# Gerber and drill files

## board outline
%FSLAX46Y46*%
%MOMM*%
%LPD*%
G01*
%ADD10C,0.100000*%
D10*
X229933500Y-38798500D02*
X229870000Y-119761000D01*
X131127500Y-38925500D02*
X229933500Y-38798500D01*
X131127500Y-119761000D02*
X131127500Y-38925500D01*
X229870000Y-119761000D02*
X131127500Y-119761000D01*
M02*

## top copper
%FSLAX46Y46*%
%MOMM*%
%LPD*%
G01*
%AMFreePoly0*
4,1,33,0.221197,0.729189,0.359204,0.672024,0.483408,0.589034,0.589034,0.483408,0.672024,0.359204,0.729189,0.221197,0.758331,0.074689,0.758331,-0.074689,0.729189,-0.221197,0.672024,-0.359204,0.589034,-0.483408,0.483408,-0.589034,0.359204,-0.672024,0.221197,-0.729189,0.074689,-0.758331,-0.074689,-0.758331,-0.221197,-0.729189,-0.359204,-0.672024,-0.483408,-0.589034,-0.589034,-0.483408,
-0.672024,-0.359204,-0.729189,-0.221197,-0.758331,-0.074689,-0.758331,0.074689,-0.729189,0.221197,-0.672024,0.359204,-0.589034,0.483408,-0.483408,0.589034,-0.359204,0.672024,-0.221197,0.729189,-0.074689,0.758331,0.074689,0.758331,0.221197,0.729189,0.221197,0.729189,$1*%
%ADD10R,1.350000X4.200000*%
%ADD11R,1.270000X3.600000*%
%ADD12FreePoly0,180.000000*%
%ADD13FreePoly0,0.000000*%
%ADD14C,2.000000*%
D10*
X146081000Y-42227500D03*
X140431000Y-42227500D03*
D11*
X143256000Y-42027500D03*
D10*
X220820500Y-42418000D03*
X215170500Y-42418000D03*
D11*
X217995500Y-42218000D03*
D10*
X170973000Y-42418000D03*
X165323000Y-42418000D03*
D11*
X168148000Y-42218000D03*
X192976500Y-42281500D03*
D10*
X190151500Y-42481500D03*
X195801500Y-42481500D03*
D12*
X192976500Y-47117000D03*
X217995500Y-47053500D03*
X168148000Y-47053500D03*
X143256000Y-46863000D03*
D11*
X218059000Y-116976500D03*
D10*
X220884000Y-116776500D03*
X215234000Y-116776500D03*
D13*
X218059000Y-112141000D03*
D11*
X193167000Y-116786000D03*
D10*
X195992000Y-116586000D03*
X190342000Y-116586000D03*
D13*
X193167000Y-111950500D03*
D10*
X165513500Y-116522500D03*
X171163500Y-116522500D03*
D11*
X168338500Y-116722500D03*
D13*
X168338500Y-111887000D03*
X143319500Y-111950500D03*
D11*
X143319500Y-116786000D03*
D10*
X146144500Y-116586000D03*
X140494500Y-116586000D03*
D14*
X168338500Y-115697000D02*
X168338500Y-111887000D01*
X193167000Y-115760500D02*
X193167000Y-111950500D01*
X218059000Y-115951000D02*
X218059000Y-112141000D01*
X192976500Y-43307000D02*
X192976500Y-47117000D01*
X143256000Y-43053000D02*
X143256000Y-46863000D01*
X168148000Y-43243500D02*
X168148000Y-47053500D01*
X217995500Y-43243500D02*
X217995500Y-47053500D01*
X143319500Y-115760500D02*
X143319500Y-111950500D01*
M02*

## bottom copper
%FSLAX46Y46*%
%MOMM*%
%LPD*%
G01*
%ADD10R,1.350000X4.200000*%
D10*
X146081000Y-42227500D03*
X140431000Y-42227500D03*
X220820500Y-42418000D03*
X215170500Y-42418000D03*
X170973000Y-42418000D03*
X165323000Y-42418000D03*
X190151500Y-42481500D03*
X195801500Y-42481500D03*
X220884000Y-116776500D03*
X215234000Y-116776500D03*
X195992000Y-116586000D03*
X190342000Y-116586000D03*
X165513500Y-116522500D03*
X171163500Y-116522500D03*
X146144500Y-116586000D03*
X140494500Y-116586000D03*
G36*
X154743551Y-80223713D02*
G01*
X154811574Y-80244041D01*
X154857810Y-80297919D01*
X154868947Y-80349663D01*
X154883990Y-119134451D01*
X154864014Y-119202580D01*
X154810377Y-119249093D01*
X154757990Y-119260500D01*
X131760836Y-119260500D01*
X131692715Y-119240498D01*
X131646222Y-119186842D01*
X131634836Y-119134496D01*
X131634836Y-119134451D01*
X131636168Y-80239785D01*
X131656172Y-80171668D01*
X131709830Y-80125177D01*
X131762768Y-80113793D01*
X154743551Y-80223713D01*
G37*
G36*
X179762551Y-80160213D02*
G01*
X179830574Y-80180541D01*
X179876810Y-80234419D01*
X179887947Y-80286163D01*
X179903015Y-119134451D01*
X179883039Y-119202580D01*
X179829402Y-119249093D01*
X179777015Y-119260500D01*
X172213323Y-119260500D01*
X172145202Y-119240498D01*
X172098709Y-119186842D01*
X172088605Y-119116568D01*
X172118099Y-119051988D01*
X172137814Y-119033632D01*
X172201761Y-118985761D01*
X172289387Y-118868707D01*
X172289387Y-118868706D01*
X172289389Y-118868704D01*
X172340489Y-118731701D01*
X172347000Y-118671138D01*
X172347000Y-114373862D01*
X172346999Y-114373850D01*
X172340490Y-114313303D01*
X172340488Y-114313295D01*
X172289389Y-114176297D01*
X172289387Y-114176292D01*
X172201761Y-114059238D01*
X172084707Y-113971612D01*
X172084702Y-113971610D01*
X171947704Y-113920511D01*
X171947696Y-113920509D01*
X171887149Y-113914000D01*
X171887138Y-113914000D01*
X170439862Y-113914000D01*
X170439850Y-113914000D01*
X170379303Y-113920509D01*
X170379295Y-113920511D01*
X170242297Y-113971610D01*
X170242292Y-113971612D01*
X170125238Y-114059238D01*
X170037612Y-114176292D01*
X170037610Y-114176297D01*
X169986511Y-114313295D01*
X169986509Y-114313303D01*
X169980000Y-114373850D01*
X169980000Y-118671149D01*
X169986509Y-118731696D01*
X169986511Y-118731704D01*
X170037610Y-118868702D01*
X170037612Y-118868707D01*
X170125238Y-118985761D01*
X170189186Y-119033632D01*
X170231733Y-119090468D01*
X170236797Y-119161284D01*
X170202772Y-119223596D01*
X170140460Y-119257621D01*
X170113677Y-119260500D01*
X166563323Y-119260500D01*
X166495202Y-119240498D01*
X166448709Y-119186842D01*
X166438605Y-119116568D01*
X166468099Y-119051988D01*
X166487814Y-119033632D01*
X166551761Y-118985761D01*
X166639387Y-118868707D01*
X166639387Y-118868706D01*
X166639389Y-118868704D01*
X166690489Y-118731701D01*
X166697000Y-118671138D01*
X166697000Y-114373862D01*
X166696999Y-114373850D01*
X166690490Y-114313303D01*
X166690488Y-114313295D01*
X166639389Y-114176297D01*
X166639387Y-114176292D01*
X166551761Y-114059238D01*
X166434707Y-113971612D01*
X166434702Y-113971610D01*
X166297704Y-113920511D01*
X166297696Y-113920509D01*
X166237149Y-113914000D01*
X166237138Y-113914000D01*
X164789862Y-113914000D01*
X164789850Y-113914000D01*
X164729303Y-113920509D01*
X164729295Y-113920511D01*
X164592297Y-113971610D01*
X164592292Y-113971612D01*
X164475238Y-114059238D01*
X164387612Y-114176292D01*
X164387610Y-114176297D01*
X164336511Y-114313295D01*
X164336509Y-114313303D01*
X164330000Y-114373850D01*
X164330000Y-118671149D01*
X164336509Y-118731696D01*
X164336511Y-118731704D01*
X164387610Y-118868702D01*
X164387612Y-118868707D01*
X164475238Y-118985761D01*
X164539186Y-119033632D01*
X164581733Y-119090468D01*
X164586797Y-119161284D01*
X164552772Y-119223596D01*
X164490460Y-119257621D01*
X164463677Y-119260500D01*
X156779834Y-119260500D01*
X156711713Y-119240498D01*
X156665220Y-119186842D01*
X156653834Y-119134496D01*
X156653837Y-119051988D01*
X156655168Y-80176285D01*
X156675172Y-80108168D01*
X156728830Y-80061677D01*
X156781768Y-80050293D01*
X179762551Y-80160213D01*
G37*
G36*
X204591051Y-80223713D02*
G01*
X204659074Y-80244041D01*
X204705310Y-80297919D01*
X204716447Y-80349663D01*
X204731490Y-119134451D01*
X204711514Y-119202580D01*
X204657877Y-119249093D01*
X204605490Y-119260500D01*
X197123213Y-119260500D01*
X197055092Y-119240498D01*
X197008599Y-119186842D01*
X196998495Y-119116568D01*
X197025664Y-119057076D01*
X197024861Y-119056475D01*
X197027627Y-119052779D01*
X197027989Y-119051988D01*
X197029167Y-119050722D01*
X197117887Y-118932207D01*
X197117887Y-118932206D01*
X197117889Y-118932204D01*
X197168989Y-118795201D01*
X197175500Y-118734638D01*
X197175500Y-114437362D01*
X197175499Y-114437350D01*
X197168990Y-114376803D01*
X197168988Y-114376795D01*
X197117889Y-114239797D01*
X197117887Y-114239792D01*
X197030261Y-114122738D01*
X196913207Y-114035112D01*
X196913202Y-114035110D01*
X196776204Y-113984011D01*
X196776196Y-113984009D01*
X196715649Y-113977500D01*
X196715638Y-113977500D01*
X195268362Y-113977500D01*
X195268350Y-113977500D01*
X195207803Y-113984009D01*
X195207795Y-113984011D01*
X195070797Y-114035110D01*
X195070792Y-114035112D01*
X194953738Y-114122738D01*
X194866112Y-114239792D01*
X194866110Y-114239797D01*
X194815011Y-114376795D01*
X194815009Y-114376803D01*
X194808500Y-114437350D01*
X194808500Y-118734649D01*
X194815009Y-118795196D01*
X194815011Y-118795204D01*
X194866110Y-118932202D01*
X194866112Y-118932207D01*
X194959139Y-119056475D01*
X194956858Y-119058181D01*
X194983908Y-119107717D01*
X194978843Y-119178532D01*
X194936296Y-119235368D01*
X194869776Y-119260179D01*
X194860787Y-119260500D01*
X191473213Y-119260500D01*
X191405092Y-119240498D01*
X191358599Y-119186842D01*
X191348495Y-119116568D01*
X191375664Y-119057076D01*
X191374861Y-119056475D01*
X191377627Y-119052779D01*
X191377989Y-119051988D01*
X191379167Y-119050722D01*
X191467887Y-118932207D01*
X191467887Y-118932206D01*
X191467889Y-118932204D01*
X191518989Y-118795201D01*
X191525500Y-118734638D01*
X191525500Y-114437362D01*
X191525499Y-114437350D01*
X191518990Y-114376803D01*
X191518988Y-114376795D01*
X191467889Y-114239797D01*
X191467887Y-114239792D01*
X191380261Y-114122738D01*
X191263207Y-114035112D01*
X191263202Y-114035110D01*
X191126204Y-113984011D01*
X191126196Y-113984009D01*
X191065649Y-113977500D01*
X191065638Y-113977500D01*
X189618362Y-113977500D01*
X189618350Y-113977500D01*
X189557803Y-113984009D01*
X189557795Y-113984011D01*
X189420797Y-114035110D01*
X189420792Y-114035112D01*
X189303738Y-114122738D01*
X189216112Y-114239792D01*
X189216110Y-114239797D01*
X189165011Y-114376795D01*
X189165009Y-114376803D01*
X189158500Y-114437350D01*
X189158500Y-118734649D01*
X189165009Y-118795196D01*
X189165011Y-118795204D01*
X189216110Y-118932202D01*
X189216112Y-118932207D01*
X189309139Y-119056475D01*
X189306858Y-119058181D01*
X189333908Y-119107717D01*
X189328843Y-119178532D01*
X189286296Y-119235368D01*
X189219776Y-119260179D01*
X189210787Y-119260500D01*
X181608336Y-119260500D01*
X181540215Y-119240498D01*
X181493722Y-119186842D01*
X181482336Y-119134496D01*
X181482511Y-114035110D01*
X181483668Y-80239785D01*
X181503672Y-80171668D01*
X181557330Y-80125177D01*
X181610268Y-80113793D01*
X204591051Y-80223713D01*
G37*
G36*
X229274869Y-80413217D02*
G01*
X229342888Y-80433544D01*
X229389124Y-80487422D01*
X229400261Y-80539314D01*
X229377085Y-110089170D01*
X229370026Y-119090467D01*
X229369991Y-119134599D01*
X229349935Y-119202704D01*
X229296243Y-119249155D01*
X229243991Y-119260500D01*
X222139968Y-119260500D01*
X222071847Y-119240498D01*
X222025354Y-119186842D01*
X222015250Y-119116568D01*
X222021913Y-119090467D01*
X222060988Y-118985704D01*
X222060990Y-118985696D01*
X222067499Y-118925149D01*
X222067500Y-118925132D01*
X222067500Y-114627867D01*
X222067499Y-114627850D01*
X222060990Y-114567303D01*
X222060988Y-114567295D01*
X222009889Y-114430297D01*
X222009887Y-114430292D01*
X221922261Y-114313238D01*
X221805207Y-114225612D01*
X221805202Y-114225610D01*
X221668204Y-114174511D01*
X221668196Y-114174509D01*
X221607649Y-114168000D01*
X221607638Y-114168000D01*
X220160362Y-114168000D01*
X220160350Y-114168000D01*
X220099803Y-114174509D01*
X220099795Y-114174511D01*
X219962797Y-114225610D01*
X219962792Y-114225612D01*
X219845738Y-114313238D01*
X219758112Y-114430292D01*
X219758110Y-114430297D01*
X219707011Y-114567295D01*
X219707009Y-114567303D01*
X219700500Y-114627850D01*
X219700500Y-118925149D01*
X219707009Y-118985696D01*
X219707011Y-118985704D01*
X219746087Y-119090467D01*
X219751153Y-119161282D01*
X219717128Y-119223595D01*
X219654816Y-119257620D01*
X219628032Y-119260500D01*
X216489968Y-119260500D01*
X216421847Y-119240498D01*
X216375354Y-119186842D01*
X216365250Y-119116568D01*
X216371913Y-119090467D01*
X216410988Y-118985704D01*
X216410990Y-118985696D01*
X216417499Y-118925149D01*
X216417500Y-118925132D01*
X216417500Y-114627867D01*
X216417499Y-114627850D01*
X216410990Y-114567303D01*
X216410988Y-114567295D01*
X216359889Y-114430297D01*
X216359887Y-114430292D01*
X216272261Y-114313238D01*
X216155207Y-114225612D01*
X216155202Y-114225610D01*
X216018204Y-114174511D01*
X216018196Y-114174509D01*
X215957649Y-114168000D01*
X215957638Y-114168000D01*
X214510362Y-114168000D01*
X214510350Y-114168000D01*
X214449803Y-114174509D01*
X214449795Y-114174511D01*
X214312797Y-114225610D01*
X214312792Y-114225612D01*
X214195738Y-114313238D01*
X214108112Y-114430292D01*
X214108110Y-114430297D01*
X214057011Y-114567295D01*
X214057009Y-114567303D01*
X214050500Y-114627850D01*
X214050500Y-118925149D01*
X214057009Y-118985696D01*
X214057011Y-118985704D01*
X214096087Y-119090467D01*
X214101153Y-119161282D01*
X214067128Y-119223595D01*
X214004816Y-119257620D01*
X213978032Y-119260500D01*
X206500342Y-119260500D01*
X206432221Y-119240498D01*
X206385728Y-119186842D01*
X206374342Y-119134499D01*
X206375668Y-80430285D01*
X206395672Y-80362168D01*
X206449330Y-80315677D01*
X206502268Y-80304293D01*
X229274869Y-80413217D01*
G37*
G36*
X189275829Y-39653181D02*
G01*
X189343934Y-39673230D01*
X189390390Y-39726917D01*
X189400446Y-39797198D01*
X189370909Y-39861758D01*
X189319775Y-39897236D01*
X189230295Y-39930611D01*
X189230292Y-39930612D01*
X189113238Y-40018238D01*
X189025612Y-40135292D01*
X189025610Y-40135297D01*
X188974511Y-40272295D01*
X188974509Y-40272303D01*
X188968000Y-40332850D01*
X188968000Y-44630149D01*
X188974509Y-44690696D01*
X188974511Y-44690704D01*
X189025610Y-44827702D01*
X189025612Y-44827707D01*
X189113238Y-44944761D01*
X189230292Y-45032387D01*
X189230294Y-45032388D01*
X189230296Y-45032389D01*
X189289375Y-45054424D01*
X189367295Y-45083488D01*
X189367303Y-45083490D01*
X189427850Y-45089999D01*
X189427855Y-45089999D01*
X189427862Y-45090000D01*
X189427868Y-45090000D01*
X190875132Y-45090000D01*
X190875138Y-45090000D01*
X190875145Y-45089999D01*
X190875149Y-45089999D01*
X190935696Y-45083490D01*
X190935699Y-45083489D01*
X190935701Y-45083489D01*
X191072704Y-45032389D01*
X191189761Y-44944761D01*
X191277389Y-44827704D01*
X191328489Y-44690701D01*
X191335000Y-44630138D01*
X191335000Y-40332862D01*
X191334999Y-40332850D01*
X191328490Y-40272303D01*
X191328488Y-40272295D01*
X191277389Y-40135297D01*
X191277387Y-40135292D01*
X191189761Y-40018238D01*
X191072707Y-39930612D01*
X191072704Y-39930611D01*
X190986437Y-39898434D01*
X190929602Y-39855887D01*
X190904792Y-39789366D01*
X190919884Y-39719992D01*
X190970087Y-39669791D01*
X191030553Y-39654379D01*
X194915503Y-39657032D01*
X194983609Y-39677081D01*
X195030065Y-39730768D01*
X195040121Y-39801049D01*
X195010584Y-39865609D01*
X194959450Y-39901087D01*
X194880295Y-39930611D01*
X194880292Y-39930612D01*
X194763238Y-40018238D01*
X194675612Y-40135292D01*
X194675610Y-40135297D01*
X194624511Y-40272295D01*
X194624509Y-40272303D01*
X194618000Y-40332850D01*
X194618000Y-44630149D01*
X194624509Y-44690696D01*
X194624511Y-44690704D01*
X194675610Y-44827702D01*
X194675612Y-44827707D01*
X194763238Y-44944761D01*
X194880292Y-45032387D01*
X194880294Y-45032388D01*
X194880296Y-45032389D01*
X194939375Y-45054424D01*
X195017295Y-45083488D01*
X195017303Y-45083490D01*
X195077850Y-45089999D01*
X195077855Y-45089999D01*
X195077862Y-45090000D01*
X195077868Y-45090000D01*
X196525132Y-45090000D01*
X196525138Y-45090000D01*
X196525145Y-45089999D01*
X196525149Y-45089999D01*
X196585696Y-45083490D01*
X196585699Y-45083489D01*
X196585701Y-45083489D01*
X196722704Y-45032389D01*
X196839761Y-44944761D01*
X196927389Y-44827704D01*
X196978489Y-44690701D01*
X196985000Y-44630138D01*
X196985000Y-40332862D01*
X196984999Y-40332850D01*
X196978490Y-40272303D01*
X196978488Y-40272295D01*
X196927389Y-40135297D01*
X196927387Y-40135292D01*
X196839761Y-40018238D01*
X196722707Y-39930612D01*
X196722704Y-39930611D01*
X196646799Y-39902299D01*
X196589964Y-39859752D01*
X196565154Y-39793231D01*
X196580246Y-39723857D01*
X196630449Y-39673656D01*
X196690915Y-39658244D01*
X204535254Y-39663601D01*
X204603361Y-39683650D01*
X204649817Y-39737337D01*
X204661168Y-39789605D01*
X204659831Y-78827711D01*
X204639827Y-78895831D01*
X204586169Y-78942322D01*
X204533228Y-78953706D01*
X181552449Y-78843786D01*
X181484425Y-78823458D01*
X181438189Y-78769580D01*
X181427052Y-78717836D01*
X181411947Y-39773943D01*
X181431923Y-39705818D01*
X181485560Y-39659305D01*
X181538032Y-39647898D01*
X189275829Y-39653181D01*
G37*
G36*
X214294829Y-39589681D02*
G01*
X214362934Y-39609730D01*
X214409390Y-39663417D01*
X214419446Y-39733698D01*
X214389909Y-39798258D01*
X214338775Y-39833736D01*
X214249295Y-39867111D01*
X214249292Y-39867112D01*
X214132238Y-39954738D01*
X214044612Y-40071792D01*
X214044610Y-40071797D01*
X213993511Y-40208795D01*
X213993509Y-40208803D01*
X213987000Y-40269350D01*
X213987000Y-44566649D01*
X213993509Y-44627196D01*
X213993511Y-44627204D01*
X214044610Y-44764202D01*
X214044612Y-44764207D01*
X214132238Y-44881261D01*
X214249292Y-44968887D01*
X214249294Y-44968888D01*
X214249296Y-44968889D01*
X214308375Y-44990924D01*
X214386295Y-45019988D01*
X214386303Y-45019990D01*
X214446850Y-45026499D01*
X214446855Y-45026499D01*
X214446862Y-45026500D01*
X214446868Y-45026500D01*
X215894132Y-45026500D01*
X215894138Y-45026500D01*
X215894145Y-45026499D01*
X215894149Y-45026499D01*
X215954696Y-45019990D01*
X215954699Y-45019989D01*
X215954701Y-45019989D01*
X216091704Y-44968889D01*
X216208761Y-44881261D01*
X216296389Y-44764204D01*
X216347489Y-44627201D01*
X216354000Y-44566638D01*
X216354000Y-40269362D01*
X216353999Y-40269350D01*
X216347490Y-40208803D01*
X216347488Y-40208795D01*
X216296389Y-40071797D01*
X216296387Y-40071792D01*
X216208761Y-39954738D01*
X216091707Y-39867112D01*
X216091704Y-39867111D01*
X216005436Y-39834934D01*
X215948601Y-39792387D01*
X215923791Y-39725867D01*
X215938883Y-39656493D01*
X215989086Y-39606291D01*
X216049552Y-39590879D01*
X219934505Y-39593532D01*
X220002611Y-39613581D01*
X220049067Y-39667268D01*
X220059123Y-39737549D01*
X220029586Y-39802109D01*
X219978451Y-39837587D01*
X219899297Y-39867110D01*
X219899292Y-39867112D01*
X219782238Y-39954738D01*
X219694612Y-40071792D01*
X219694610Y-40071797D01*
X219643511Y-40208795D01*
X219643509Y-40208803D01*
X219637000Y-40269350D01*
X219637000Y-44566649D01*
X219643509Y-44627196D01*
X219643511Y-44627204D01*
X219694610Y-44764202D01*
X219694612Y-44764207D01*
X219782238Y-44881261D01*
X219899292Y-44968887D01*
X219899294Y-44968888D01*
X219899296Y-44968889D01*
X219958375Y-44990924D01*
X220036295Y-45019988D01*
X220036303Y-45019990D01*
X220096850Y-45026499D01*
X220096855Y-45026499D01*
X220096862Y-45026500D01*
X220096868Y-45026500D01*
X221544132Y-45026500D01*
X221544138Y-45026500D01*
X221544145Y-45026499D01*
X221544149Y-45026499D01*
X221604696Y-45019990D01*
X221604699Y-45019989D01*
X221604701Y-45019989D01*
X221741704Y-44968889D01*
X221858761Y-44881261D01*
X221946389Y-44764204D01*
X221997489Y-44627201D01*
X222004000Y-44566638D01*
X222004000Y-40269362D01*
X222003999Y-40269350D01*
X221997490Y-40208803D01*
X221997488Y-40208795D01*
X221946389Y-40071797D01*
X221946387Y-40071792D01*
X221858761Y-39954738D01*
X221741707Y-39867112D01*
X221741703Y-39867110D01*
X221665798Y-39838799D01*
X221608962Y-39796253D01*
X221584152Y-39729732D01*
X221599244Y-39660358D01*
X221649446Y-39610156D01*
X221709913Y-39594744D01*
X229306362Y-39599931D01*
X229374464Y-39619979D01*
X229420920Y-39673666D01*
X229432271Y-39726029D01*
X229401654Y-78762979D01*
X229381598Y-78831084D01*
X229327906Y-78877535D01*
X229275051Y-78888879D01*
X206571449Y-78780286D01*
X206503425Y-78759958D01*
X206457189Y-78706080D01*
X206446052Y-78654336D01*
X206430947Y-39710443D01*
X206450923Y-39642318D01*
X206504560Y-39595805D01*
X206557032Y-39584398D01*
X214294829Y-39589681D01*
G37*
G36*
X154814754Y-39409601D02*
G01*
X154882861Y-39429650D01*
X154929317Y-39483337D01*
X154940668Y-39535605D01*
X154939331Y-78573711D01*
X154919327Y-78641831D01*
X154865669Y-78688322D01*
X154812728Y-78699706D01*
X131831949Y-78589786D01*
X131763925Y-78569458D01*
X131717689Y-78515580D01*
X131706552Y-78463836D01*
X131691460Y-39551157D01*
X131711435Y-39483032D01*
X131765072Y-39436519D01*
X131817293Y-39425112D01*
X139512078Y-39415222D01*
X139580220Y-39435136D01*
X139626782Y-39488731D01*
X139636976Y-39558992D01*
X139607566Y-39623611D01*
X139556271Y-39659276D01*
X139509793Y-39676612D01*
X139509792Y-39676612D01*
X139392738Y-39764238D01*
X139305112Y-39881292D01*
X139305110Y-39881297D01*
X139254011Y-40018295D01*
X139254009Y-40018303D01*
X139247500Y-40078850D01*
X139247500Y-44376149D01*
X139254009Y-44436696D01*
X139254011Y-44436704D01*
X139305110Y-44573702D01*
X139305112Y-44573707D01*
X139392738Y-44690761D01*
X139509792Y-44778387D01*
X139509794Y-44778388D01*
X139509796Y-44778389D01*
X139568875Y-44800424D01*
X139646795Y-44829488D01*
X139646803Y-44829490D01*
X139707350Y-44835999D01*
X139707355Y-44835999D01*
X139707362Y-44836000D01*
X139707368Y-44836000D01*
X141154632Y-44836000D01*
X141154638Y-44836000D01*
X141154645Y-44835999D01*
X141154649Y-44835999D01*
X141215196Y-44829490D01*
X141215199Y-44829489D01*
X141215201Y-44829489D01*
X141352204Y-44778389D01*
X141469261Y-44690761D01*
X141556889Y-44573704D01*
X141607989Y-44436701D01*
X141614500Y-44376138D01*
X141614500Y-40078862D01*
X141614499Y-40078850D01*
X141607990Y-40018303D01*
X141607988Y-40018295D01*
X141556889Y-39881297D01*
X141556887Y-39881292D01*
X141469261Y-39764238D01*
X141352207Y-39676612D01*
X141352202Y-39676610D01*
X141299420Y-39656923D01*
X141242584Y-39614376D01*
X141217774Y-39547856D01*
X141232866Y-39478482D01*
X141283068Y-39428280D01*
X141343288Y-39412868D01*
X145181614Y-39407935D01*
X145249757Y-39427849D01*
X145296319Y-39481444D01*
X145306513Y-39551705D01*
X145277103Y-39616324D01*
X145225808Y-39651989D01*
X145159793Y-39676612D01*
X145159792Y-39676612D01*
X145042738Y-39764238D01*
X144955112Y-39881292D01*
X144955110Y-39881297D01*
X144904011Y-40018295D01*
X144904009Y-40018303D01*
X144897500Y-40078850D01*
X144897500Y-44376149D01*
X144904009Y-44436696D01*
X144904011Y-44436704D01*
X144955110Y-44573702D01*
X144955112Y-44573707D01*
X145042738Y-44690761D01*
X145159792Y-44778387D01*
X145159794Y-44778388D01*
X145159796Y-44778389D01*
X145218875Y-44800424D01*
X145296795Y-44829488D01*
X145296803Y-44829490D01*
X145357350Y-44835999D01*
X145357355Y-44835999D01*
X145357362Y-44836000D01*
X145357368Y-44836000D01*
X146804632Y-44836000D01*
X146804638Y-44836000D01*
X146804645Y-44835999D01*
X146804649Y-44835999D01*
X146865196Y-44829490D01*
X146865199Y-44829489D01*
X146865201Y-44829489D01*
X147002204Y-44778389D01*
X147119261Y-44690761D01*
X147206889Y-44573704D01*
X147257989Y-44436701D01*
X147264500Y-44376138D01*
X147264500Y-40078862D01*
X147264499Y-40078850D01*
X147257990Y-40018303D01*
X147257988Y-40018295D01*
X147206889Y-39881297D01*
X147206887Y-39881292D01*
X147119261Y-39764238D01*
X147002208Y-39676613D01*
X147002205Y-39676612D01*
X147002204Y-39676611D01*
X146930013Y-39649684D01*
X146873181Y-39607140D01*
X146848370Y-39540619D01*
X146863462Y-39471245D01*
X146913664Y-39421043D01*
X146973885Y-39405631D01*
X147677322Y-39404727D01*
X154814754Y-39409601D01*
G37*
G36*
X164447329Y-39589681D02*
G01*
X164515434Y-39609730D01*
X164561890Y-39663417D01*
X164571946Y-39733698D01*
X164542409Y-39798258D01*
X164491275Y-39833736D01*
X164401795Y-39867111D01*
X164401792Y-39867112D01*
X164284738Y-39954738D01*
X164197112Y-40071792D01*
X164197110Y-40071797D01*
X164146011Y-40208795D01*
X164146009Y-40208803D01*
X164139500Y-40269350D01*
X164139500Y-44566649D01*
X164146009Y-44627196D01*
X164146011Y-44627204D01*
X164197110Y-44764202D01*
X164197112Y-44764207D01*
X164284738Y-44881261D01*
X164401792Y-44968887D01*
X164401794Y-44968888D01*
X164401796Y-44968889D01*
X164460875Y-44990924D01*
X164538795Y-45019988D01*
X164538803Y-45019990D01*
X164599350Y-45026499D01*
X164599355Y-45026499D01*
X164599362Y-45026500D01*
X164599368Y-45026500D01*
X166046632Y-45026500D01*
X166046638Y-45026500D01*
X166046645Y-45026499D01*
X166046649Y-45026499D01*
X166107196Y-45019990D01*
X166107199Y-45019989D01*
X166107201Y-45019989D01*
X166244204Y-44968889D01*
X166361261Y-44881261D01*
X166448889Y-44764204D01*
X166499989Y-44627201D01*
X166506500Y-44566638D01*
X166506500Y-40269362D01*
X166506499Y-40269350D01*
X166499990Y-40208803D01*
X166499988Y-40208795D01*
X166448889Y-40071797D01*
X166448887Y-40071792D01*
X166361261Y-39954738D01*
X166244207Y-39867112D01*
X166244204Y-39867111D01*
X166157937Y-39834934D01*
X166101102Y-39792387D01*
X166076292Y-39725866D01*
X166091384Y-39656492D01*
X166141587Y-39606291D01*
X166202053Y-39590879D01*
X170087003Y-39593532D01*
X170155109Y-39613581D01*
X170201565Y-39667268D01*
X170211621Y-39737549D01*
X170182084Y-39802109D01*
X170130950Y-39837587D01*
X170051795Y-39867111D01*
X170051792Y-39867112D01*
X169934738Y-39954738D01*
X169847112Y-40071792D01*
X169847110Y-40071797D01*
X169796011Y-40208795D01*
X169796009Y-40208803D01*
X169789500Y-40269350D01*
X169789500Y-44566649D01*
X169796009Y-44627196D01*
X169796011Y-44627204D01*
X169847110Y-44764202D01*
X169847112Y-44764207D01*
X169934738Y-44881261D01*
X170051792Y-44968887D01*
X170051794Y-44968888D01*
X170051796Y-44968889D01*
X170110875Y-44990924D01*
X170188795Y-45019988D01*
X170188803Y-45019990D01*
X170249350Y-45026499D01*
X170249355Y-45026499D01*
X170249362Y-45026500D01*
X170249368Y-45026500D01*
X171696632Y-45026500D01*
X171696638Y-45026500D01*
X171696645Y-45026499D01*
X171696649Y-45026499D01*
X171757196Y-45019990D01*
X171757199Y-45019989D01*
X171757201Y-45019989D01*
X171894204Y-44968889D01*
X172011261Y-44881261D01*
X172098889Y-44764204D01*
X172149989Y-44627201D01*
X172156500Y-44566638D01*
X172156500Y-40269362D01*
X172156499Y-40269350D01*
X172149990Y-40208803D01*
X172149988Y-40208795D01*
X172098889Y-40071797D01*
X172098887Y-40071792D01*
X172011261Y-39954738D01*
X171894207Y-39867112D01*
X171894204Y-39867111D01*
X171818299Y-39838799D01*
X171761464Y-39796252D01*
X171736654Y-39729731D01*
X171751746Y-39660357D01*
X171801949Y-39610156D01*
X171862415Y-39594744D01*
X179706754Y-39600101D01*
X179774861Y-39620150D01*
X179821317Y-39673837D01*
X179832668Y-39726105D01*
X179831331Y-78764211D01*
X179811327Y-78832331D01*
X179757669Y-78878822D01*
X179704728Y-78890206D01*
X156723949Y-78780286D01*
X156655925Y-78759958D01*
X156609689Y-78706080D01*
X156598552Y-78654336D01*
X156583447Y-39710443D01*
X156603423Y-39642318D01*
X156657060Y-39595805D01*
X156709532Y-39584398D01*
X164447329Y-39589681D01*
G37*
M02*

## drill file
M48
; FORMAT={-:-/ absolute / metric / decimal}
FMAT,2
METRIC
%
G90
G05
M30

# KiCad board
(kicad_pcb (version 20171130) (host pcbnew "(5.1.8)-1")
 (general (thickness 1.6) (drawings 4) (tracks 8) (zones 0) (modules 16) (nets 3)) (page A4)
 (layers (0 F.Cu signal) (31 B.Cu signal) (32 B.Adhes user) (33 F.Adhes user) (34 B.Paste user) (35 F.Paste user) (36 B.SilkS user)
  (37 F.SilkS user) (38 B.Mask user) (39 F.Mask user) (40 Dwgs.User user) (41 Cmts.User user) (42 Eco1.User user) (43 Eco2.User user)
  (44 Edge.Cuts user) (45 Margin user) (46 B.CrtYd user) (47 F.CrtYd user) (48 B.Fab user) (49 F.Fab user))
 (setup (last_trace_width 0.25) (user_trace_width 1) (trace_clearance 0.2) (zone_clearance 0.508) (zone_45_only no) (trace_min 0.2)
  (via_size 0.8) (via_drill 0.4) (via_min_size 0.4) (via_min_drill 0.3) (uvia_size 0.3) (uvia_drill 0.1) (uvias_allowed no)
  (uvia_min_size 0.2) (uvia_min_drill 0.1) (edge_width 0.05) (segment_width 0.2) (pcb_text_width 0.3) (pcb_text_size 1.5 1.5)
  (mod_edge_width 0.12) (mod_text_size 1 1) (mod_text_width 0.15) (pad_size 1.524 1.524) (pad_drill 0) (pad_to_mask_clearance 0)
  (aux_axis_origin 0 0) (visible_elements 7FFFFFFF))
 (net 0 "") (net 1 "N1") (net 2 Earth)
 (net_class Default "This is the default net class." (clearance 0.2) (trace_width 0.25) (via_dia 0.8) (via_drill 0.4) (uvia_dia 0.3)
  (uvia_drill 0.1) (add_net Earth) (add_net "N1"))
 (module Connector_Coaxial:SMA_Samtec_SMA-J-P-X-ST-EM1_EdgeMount (layer F.Cu) (at 143.256 42.2275 180)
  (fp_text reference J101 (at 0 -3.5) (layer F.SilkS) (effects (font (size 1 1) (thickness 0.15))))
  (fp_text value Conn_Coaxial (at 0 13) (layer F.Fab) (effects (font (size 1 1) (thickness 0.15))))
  (pad 2 smd rect (at -2.825 0 180) (size 1.35 4.2) (layers B.Cu B.Paste B.Mask))
  (pad 2 smd rect (at 2.825 0 180) (size 1.35 4.2) (layers B.Cu B.Paste B.Mask))
  (pad 2 smd rect (at -2.825 0 180) (size 1.35 4.2) (layers F.Cu F.Paste F.Mask))
  (pad 2 smd rect (at 2.825 0 180) (size 1.35 4.2) (layers F.Cu F.Paste F.Mask))
  (pad 1 smd rect (at 0 0.2 180) (size 1.27 3.6) (layers F.Cu F.Paste F.Mask)))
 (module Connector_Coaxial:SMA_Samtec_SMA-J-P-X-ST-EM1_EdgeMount (layer F.Cu) (at 217.9955 42.418 180)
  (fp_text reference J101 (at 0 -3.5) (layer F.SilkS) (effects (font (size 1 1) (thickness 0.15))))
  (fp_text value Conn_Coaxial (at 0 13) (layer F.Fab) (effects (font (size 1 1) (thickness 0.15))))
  (pad 2 smd rect (at -2.825 0 180) (size 1.35 4.2) (layers B.Cu B.Paste B.Mask))
  (pad 2 smd rect (at 2.825 0 180) (size 1.35 4.2) (layers B.Cu B.Paste B.Mask))
  (pad 2 smd rect (at -2.825 0 180) (size 1.35 4.2) (layers F.Cu F.Paste F.Mask))
  (pad 2 smd rect (at 2.825 0 180) (size 1.35 4.2) (layers F.Cu F.Paste F.Mask))
  (pad 1 smd rect (at 0 0.2 180) (size 1.27 3.6) (layers F.Cu F.Paste F.Mask)))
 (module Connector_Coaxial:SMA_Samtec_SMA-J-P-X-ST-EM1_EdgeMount (layer F.Cu) (at 168.148 42.418 180)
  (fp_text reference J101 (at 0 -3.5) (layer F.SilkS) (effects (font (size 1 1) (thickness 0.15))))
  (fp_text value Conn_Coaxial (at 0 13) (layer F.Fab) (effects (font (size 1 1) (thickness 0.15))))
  (pad 2 smd rect (at -2.825 0 180) (size 1.35 4.2) (layers B.Cu B.Paste B.Mask))
  (pad 2 smd rect (at 2.825 0 180) (size 1.35 4.2) (layers B.Cu B.Paste B.Mask))
  (pad 2 smd rect (at -2.825 0 180) (size 1.35 4.2) (layers F.Cu F.Paste F.Mask))
  (pad 2 smd rect (at 2.825 0 180) (size 1.35 4.2) (layers F.Cu F.Paste F.Mask))
  (pad 1 smd rect (at 0 0.2 180) (size 1.27 3.6) (layers F.Cu F.Paste F.Mask)))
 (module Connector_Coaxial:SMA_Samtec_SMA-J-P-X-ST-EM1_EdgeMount (layer F.Cu) (at 192.9765 42.4815 180)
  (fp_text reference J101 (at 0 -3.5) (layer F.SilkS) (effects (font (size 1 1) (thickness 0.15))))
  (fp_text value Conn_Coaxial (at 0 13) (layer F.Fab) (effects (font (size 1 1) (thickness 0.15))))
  (pad 1 smd rect (at 0 0.2 180) (size 1.27 3.6) (layers F.Cu F.Paste F.Mask))
  (pad 2 smd rect (at 2.825 0 180) (size 1.35 4.2) (layers F.Cu F.Paste F.Mask))
  (pad 2 smd rect (at -2.825 0 180) (size 1.35 4.2) (layers F.Cu F.Paste F.Mask))
  (pad 2 smd rect (at 2.825 0 180) (size 1.35 4.2) (layers B.Cu B.Paste B.Mask))
  (pad 2 smd rect (at -2.825 0 180) (size 1.35 4.2) (layers B.Cu B.Paste B.Mask)))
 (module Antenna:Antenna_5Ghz (layer F.Cu) (at 192.659 63.1825 180)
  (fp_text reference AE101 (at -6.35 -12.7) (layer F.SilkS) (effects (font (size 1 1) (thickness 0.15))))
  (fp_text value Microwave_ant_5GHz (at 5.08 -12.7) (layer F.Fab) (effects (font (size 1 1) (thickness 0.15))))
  (pad 1 smd custom (at -0.3175 16.0655 180) (size 1.524 1.524) (layers F.Cu F.Paste F.Mask) (options (clearance outline) (anchor circle))
   (primitives)))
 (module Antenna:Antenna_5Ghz (layer F.Cu) (at 217.678 63.119 180)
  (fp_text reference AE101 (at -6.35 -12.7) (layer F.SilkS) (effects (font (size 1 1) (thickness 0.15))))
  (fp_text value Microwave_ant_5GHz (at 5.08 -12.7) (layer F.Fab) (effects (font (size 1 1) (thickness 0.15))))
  (pad 1 smd custom (at -0.3175 16.0655 180) (size 1.524 1.524) (layers F.Cu F.Paste F.Mask) (options (clearance outline) (anchor circle))
   (primitives)))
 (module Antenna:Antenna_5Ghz (layer F.Cu) (at 167.8305 63.119 180)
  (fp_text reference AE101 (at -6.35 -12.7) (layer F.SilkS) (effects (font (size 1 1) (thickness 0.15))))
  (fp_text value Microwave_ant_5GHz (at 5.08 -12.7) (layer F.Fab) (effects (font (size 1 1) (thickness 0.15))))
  (pad 1 smd custom (at -0.3175 16.0655 180) (size 1.524 1.524) (layers F.Cu F.Paste F.Mask) (options (clearance outline) (anchor circle))
   (primitives)))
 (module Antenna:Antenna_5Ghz (layer F.Cu) (at 142.9385 62.9285 180)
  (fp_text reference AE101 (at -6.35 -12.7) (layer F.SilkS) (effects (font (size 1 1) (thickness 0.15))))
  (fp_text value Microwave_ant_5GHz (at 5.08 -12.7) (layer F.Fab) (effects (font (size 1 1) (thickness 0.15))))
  (pad 1 smd custom (at -0.3175 16.0655 180) (size 1.524 1.524) (layers F.Cu F.Paste F.Mask) (options (clearance outline) (anchor circle))
   (primitives)))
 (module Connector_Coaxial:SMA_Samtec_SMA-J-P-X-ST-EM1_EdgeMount (layer F.Cu) (at 218.059 116.7765)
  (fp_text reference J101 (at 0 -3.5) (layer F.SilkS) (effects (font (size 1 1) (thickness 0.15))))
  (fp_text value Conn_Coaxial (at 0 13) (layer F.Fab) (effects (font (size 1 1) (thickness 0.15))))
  (pad 1 smd rect (at 0 0.2) (size 1.27 3.6) (layers F.Cu F.Paste F.Mask))
  (pad 2 smd rect (at 2.825 0) (size 1.35 4.2) (layers F.Cu F.Paste F.Mask))
  (pad 2 smd rect (at -2.825 0) (size 1.35 4.2) (layers F.Cu F.Paste F.Mask))
  (pad 2 smd rect (at 2.825 0) (size 1.35 4.2) (layers B.Cu B.Paste B.Mask))
  (pad 2 smd rect (at -2.825 0) (size 1.35 4.2) (layers B.Cu B.Paste B.Mask)))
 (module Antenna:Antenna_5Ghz (layer F.Cu) (at 218.3765 96.0755)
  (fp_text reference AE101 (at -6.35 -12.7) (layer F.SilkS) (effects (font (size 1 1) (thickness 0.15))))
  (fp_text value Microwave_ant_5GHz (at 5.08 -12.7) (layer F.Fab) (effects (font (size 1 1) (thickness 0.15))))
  (pad 1 smd custom (at -0.3175 16.0655) (size 1.524 1.524) (layers F.Cu F.Paste F.Mask) (options (clearance outline) (anchor circle))
   (primitives)))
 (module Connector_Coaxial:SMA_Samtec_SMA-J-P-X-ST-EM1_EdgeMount (layer F.Cu) (at 193.167 116.586)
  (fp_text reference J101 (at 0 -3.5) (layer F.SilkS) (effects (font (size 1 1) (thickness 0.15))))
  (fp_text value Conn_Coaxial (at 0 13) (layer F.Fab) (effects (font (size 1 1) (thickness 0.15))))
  (pad 1 smd rect (at 0 0.2) (size 1.27 3.6) (layers F.Cu F.Paste F.Mask))
  (pad 2 smd rect (at 2.825 0) (size 1.35 4.2) (layers F.Cu F.Paste F.Mask))
  (pad 2 smd rect (at -2.825 0) (size 1.35 4.2) (layers F.Cu F.Paste F.Mask))
  (pad 2 smd rect (at 2.825 0) (size 1.35 4.2) (layers B.Cu B.Paste B.Mask))
  (pad 2 smd rect (at -2.825 0) (size 1.35 4.2) (layers B.Cu B.Paste B.Mask)))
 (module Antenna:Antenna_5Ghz (layer F.Cu) (at 193.4845 95.885)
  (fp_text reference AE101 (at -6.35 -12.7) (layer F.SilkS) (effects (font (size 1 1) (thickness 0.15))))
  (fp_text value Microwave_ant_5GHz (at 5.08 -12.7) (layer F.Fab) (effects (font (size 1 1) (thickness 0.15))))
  (pad 1 smd custom (at -0.3175 16.0655) (size 1.524 1.524) (layers F.Cu F.Paste F.Mask) (options (clearance outline) (anchor circle))
   (primitives)))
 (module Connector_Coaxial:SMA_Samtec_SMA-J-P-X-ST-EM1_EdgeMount (layer F.Cu) (at 168.3385 116.5225)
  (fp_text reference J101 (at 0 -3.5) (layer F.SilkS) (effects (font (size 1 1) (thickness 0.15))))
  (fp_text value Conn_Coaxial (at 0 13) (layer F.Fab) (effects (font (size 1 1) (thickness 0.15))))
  (pad 2 smd rect (at -2.825 0) (size 1.35 4.2) (layers B.Cu B.Paste B.Mask))
  (pad 2 smd rect (at 2.825 0) (size 1.35 4.2) (layers B.Cu B.Paste B.Mask))
  (pad 2 smd rect (at -2.825 0) (size 1.35 4.2) (layers F.Cu F.Paste F.Mask))
  (pad 2 smd rect (at 2.825 0) (size 1.35 4.2) (layers F.Cu F.Paste F.Mask))
  (pad 1 smd rect (at 0 0.2) (size 1.27 3.6) (layers F.Cu F.Paste F.Mask)))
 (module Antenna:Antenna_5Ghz (layer F.Cu) (at 168.656 95.8215)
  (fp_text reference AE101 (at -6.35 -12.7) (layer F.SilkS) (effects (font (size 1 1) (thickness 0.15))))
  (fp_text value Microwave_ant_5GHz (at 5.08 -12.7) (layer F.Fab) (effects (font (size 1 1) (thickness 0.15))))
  (pad 1 smd custom (at -0.3175 16.0655) (size 1.524 1.524) (layers F.Cu F.Paste F.Mask) (options (clearance outline) (anchor circle))
   (primitives)))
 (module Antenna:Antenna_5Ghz (layer F.Cu) (at 143.637 95.885)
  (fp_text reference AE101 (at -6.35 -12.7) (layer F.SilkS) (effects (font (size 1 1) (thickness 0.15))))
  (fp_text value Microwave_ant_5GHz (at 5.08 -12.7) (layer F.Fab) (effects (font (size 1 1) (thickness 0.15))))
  (pad 1 smd custom (at -0.3175 16.0655) (size 1.524 1.524) (layers F.Cu F.Paste F.Mask) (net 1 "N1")
   (options (clearance outline) (anchor circle)) (primitives)))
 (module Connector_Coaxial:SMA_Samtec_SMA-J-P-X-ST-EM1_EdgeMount (layer F.Cu) (at 143.3195 116.586)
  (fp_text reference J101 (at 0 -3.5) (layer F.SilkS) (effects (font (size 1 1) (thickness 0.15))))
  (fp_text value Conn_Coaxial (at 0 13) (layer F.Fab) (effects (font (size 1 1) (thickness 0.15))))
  (pad 1 smd rect (at 0 0.2) (size 1.27 3.6) (layers F.Cu F.Paste F.Mask) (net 1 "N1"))
  (pad 2 smd rect (at 2.825 0) (size 1.35 4.2) (layers F.Cu F.Paste F.Mask) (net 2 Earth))
  (pad 2 smd rect (at -2.825 0) (size 1.35 4.2) (layers F.Cu F.Paste F.Mask) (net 2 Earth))
  (pad 2 smd rect (at 2.825 0) (size 1.35 4.2) (layers B.Cu B.Paste B.Mask) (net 2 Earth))
  (pad 2 smd rect (at -2.825 0) (size 1.35 4.2) (layers B.Cu B.Paste B.Mask) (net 2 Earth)))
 (gr_line (start 229.9335 38.7985) (end 229.87 119.761) (layer Edge.Cuts) (width 0.1))
 (gr_line (start 131.1275 38.9255) (end 229.9335 38.7985) (layer Edge.Cuts) (width 0.1))
 (gr_line (start 131.1275 119.761) (end 131.1275 38.9255) (layer Edge.Cuts) (width 0.1))
 (gr_line (start 229.87 119.761) (end 131.1275 119.761) (layer Edge.Cuts) (width 0.1))
 (segment (start 168.3385 115.697) (end 168.3385 111.887) (width 2) (layer F.Cu) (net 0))
 (segment (start 193.167 115.7605) (end 193.167 111.9505) (width 2) (layer F.Cu) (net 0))
 (segment (start 218.059 115.951) (end 218.059 112.141) (width 2) (layer F.Cu) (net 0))
 (segment (start 192.9765 43.307) (end 192.9765 47.117) (width 2) (layer F.Cu) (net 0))
 (segment (start 143.256 43.053) (end 143.256 46.863) (width 2) (layer F.Cu) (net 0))
 (segment (start 168.148 43.2435) (end 168.148 47.0535) (width 2) (layer F.Cu) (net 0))
 (segment (start 217.9955 43.2435) (end 217.9955 47.0535) (width 2) (layer F.Cu) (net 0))
 (segment (start 143.3195 115.7605) (end 143.3195 111.9505) (width 2) (layer F.Cu) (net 1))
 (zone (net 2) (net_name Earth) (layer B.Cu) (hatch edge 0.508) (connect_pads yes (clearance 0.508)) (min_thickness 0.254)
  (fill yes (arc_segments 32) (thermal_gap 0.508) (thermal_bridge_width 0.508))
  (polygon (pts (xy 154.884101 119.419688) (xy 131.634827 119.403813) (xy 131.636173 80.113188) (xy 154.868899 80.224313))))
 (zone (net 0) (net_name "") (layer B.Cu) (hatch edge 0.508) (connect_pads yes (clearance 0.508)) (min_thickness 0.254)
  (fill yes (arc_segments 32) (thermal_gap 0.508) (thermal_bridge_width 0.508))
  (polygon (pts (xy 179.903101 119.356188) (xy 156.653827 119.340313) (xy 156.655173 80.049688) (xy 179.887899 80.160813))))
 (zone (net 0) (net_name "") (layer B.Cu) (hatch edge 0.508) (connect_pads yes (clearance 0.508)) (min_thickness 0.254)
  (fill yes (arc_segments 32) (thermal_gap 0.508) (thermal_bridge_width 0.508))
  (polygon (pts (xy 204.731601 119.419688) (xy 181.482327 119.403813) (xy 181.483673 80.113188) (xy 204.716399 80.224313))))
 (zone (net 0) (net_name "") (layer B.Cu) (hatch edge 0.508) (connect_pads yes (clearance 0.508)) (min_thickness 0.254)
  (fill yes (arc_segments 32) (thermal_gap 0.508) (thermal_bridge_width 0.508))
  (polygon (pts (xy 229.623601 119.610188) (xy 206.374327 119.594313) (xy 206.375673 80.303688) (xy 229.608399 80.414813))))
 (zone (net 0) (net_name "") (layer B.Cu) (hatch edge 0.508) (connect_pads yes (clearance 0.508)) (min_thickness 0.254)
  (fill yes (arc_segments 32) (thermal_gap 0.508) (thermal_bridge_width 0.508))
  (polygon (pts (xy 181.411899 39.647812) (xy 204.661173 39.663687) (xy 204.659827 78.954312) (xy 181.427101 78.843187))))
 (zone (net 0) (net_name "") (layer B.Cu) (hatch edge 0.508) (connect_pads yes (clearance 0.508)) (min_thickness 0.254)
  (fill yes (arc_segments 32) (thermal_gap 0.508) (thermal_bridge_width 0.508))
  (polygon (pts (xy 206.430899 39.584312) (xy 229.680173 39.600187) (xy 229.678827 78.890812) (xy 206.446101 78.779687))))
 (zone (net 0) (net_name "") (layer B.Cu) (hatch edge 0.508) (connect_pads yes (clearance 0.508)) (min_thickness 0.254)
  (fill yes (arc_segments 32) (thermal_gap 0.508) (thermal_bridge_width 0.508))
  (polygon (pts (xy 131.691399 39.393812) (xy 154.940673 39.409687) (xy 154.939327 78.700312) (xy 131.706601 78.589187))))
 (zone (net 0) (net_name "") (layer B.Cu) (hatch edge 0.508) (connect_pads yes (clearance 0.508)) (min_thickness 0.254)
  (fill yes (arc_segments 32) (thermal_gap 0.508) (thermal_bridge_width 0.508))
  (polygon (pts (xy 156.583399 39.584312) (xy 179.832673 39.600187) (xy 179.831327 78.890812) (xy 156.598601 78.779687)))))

